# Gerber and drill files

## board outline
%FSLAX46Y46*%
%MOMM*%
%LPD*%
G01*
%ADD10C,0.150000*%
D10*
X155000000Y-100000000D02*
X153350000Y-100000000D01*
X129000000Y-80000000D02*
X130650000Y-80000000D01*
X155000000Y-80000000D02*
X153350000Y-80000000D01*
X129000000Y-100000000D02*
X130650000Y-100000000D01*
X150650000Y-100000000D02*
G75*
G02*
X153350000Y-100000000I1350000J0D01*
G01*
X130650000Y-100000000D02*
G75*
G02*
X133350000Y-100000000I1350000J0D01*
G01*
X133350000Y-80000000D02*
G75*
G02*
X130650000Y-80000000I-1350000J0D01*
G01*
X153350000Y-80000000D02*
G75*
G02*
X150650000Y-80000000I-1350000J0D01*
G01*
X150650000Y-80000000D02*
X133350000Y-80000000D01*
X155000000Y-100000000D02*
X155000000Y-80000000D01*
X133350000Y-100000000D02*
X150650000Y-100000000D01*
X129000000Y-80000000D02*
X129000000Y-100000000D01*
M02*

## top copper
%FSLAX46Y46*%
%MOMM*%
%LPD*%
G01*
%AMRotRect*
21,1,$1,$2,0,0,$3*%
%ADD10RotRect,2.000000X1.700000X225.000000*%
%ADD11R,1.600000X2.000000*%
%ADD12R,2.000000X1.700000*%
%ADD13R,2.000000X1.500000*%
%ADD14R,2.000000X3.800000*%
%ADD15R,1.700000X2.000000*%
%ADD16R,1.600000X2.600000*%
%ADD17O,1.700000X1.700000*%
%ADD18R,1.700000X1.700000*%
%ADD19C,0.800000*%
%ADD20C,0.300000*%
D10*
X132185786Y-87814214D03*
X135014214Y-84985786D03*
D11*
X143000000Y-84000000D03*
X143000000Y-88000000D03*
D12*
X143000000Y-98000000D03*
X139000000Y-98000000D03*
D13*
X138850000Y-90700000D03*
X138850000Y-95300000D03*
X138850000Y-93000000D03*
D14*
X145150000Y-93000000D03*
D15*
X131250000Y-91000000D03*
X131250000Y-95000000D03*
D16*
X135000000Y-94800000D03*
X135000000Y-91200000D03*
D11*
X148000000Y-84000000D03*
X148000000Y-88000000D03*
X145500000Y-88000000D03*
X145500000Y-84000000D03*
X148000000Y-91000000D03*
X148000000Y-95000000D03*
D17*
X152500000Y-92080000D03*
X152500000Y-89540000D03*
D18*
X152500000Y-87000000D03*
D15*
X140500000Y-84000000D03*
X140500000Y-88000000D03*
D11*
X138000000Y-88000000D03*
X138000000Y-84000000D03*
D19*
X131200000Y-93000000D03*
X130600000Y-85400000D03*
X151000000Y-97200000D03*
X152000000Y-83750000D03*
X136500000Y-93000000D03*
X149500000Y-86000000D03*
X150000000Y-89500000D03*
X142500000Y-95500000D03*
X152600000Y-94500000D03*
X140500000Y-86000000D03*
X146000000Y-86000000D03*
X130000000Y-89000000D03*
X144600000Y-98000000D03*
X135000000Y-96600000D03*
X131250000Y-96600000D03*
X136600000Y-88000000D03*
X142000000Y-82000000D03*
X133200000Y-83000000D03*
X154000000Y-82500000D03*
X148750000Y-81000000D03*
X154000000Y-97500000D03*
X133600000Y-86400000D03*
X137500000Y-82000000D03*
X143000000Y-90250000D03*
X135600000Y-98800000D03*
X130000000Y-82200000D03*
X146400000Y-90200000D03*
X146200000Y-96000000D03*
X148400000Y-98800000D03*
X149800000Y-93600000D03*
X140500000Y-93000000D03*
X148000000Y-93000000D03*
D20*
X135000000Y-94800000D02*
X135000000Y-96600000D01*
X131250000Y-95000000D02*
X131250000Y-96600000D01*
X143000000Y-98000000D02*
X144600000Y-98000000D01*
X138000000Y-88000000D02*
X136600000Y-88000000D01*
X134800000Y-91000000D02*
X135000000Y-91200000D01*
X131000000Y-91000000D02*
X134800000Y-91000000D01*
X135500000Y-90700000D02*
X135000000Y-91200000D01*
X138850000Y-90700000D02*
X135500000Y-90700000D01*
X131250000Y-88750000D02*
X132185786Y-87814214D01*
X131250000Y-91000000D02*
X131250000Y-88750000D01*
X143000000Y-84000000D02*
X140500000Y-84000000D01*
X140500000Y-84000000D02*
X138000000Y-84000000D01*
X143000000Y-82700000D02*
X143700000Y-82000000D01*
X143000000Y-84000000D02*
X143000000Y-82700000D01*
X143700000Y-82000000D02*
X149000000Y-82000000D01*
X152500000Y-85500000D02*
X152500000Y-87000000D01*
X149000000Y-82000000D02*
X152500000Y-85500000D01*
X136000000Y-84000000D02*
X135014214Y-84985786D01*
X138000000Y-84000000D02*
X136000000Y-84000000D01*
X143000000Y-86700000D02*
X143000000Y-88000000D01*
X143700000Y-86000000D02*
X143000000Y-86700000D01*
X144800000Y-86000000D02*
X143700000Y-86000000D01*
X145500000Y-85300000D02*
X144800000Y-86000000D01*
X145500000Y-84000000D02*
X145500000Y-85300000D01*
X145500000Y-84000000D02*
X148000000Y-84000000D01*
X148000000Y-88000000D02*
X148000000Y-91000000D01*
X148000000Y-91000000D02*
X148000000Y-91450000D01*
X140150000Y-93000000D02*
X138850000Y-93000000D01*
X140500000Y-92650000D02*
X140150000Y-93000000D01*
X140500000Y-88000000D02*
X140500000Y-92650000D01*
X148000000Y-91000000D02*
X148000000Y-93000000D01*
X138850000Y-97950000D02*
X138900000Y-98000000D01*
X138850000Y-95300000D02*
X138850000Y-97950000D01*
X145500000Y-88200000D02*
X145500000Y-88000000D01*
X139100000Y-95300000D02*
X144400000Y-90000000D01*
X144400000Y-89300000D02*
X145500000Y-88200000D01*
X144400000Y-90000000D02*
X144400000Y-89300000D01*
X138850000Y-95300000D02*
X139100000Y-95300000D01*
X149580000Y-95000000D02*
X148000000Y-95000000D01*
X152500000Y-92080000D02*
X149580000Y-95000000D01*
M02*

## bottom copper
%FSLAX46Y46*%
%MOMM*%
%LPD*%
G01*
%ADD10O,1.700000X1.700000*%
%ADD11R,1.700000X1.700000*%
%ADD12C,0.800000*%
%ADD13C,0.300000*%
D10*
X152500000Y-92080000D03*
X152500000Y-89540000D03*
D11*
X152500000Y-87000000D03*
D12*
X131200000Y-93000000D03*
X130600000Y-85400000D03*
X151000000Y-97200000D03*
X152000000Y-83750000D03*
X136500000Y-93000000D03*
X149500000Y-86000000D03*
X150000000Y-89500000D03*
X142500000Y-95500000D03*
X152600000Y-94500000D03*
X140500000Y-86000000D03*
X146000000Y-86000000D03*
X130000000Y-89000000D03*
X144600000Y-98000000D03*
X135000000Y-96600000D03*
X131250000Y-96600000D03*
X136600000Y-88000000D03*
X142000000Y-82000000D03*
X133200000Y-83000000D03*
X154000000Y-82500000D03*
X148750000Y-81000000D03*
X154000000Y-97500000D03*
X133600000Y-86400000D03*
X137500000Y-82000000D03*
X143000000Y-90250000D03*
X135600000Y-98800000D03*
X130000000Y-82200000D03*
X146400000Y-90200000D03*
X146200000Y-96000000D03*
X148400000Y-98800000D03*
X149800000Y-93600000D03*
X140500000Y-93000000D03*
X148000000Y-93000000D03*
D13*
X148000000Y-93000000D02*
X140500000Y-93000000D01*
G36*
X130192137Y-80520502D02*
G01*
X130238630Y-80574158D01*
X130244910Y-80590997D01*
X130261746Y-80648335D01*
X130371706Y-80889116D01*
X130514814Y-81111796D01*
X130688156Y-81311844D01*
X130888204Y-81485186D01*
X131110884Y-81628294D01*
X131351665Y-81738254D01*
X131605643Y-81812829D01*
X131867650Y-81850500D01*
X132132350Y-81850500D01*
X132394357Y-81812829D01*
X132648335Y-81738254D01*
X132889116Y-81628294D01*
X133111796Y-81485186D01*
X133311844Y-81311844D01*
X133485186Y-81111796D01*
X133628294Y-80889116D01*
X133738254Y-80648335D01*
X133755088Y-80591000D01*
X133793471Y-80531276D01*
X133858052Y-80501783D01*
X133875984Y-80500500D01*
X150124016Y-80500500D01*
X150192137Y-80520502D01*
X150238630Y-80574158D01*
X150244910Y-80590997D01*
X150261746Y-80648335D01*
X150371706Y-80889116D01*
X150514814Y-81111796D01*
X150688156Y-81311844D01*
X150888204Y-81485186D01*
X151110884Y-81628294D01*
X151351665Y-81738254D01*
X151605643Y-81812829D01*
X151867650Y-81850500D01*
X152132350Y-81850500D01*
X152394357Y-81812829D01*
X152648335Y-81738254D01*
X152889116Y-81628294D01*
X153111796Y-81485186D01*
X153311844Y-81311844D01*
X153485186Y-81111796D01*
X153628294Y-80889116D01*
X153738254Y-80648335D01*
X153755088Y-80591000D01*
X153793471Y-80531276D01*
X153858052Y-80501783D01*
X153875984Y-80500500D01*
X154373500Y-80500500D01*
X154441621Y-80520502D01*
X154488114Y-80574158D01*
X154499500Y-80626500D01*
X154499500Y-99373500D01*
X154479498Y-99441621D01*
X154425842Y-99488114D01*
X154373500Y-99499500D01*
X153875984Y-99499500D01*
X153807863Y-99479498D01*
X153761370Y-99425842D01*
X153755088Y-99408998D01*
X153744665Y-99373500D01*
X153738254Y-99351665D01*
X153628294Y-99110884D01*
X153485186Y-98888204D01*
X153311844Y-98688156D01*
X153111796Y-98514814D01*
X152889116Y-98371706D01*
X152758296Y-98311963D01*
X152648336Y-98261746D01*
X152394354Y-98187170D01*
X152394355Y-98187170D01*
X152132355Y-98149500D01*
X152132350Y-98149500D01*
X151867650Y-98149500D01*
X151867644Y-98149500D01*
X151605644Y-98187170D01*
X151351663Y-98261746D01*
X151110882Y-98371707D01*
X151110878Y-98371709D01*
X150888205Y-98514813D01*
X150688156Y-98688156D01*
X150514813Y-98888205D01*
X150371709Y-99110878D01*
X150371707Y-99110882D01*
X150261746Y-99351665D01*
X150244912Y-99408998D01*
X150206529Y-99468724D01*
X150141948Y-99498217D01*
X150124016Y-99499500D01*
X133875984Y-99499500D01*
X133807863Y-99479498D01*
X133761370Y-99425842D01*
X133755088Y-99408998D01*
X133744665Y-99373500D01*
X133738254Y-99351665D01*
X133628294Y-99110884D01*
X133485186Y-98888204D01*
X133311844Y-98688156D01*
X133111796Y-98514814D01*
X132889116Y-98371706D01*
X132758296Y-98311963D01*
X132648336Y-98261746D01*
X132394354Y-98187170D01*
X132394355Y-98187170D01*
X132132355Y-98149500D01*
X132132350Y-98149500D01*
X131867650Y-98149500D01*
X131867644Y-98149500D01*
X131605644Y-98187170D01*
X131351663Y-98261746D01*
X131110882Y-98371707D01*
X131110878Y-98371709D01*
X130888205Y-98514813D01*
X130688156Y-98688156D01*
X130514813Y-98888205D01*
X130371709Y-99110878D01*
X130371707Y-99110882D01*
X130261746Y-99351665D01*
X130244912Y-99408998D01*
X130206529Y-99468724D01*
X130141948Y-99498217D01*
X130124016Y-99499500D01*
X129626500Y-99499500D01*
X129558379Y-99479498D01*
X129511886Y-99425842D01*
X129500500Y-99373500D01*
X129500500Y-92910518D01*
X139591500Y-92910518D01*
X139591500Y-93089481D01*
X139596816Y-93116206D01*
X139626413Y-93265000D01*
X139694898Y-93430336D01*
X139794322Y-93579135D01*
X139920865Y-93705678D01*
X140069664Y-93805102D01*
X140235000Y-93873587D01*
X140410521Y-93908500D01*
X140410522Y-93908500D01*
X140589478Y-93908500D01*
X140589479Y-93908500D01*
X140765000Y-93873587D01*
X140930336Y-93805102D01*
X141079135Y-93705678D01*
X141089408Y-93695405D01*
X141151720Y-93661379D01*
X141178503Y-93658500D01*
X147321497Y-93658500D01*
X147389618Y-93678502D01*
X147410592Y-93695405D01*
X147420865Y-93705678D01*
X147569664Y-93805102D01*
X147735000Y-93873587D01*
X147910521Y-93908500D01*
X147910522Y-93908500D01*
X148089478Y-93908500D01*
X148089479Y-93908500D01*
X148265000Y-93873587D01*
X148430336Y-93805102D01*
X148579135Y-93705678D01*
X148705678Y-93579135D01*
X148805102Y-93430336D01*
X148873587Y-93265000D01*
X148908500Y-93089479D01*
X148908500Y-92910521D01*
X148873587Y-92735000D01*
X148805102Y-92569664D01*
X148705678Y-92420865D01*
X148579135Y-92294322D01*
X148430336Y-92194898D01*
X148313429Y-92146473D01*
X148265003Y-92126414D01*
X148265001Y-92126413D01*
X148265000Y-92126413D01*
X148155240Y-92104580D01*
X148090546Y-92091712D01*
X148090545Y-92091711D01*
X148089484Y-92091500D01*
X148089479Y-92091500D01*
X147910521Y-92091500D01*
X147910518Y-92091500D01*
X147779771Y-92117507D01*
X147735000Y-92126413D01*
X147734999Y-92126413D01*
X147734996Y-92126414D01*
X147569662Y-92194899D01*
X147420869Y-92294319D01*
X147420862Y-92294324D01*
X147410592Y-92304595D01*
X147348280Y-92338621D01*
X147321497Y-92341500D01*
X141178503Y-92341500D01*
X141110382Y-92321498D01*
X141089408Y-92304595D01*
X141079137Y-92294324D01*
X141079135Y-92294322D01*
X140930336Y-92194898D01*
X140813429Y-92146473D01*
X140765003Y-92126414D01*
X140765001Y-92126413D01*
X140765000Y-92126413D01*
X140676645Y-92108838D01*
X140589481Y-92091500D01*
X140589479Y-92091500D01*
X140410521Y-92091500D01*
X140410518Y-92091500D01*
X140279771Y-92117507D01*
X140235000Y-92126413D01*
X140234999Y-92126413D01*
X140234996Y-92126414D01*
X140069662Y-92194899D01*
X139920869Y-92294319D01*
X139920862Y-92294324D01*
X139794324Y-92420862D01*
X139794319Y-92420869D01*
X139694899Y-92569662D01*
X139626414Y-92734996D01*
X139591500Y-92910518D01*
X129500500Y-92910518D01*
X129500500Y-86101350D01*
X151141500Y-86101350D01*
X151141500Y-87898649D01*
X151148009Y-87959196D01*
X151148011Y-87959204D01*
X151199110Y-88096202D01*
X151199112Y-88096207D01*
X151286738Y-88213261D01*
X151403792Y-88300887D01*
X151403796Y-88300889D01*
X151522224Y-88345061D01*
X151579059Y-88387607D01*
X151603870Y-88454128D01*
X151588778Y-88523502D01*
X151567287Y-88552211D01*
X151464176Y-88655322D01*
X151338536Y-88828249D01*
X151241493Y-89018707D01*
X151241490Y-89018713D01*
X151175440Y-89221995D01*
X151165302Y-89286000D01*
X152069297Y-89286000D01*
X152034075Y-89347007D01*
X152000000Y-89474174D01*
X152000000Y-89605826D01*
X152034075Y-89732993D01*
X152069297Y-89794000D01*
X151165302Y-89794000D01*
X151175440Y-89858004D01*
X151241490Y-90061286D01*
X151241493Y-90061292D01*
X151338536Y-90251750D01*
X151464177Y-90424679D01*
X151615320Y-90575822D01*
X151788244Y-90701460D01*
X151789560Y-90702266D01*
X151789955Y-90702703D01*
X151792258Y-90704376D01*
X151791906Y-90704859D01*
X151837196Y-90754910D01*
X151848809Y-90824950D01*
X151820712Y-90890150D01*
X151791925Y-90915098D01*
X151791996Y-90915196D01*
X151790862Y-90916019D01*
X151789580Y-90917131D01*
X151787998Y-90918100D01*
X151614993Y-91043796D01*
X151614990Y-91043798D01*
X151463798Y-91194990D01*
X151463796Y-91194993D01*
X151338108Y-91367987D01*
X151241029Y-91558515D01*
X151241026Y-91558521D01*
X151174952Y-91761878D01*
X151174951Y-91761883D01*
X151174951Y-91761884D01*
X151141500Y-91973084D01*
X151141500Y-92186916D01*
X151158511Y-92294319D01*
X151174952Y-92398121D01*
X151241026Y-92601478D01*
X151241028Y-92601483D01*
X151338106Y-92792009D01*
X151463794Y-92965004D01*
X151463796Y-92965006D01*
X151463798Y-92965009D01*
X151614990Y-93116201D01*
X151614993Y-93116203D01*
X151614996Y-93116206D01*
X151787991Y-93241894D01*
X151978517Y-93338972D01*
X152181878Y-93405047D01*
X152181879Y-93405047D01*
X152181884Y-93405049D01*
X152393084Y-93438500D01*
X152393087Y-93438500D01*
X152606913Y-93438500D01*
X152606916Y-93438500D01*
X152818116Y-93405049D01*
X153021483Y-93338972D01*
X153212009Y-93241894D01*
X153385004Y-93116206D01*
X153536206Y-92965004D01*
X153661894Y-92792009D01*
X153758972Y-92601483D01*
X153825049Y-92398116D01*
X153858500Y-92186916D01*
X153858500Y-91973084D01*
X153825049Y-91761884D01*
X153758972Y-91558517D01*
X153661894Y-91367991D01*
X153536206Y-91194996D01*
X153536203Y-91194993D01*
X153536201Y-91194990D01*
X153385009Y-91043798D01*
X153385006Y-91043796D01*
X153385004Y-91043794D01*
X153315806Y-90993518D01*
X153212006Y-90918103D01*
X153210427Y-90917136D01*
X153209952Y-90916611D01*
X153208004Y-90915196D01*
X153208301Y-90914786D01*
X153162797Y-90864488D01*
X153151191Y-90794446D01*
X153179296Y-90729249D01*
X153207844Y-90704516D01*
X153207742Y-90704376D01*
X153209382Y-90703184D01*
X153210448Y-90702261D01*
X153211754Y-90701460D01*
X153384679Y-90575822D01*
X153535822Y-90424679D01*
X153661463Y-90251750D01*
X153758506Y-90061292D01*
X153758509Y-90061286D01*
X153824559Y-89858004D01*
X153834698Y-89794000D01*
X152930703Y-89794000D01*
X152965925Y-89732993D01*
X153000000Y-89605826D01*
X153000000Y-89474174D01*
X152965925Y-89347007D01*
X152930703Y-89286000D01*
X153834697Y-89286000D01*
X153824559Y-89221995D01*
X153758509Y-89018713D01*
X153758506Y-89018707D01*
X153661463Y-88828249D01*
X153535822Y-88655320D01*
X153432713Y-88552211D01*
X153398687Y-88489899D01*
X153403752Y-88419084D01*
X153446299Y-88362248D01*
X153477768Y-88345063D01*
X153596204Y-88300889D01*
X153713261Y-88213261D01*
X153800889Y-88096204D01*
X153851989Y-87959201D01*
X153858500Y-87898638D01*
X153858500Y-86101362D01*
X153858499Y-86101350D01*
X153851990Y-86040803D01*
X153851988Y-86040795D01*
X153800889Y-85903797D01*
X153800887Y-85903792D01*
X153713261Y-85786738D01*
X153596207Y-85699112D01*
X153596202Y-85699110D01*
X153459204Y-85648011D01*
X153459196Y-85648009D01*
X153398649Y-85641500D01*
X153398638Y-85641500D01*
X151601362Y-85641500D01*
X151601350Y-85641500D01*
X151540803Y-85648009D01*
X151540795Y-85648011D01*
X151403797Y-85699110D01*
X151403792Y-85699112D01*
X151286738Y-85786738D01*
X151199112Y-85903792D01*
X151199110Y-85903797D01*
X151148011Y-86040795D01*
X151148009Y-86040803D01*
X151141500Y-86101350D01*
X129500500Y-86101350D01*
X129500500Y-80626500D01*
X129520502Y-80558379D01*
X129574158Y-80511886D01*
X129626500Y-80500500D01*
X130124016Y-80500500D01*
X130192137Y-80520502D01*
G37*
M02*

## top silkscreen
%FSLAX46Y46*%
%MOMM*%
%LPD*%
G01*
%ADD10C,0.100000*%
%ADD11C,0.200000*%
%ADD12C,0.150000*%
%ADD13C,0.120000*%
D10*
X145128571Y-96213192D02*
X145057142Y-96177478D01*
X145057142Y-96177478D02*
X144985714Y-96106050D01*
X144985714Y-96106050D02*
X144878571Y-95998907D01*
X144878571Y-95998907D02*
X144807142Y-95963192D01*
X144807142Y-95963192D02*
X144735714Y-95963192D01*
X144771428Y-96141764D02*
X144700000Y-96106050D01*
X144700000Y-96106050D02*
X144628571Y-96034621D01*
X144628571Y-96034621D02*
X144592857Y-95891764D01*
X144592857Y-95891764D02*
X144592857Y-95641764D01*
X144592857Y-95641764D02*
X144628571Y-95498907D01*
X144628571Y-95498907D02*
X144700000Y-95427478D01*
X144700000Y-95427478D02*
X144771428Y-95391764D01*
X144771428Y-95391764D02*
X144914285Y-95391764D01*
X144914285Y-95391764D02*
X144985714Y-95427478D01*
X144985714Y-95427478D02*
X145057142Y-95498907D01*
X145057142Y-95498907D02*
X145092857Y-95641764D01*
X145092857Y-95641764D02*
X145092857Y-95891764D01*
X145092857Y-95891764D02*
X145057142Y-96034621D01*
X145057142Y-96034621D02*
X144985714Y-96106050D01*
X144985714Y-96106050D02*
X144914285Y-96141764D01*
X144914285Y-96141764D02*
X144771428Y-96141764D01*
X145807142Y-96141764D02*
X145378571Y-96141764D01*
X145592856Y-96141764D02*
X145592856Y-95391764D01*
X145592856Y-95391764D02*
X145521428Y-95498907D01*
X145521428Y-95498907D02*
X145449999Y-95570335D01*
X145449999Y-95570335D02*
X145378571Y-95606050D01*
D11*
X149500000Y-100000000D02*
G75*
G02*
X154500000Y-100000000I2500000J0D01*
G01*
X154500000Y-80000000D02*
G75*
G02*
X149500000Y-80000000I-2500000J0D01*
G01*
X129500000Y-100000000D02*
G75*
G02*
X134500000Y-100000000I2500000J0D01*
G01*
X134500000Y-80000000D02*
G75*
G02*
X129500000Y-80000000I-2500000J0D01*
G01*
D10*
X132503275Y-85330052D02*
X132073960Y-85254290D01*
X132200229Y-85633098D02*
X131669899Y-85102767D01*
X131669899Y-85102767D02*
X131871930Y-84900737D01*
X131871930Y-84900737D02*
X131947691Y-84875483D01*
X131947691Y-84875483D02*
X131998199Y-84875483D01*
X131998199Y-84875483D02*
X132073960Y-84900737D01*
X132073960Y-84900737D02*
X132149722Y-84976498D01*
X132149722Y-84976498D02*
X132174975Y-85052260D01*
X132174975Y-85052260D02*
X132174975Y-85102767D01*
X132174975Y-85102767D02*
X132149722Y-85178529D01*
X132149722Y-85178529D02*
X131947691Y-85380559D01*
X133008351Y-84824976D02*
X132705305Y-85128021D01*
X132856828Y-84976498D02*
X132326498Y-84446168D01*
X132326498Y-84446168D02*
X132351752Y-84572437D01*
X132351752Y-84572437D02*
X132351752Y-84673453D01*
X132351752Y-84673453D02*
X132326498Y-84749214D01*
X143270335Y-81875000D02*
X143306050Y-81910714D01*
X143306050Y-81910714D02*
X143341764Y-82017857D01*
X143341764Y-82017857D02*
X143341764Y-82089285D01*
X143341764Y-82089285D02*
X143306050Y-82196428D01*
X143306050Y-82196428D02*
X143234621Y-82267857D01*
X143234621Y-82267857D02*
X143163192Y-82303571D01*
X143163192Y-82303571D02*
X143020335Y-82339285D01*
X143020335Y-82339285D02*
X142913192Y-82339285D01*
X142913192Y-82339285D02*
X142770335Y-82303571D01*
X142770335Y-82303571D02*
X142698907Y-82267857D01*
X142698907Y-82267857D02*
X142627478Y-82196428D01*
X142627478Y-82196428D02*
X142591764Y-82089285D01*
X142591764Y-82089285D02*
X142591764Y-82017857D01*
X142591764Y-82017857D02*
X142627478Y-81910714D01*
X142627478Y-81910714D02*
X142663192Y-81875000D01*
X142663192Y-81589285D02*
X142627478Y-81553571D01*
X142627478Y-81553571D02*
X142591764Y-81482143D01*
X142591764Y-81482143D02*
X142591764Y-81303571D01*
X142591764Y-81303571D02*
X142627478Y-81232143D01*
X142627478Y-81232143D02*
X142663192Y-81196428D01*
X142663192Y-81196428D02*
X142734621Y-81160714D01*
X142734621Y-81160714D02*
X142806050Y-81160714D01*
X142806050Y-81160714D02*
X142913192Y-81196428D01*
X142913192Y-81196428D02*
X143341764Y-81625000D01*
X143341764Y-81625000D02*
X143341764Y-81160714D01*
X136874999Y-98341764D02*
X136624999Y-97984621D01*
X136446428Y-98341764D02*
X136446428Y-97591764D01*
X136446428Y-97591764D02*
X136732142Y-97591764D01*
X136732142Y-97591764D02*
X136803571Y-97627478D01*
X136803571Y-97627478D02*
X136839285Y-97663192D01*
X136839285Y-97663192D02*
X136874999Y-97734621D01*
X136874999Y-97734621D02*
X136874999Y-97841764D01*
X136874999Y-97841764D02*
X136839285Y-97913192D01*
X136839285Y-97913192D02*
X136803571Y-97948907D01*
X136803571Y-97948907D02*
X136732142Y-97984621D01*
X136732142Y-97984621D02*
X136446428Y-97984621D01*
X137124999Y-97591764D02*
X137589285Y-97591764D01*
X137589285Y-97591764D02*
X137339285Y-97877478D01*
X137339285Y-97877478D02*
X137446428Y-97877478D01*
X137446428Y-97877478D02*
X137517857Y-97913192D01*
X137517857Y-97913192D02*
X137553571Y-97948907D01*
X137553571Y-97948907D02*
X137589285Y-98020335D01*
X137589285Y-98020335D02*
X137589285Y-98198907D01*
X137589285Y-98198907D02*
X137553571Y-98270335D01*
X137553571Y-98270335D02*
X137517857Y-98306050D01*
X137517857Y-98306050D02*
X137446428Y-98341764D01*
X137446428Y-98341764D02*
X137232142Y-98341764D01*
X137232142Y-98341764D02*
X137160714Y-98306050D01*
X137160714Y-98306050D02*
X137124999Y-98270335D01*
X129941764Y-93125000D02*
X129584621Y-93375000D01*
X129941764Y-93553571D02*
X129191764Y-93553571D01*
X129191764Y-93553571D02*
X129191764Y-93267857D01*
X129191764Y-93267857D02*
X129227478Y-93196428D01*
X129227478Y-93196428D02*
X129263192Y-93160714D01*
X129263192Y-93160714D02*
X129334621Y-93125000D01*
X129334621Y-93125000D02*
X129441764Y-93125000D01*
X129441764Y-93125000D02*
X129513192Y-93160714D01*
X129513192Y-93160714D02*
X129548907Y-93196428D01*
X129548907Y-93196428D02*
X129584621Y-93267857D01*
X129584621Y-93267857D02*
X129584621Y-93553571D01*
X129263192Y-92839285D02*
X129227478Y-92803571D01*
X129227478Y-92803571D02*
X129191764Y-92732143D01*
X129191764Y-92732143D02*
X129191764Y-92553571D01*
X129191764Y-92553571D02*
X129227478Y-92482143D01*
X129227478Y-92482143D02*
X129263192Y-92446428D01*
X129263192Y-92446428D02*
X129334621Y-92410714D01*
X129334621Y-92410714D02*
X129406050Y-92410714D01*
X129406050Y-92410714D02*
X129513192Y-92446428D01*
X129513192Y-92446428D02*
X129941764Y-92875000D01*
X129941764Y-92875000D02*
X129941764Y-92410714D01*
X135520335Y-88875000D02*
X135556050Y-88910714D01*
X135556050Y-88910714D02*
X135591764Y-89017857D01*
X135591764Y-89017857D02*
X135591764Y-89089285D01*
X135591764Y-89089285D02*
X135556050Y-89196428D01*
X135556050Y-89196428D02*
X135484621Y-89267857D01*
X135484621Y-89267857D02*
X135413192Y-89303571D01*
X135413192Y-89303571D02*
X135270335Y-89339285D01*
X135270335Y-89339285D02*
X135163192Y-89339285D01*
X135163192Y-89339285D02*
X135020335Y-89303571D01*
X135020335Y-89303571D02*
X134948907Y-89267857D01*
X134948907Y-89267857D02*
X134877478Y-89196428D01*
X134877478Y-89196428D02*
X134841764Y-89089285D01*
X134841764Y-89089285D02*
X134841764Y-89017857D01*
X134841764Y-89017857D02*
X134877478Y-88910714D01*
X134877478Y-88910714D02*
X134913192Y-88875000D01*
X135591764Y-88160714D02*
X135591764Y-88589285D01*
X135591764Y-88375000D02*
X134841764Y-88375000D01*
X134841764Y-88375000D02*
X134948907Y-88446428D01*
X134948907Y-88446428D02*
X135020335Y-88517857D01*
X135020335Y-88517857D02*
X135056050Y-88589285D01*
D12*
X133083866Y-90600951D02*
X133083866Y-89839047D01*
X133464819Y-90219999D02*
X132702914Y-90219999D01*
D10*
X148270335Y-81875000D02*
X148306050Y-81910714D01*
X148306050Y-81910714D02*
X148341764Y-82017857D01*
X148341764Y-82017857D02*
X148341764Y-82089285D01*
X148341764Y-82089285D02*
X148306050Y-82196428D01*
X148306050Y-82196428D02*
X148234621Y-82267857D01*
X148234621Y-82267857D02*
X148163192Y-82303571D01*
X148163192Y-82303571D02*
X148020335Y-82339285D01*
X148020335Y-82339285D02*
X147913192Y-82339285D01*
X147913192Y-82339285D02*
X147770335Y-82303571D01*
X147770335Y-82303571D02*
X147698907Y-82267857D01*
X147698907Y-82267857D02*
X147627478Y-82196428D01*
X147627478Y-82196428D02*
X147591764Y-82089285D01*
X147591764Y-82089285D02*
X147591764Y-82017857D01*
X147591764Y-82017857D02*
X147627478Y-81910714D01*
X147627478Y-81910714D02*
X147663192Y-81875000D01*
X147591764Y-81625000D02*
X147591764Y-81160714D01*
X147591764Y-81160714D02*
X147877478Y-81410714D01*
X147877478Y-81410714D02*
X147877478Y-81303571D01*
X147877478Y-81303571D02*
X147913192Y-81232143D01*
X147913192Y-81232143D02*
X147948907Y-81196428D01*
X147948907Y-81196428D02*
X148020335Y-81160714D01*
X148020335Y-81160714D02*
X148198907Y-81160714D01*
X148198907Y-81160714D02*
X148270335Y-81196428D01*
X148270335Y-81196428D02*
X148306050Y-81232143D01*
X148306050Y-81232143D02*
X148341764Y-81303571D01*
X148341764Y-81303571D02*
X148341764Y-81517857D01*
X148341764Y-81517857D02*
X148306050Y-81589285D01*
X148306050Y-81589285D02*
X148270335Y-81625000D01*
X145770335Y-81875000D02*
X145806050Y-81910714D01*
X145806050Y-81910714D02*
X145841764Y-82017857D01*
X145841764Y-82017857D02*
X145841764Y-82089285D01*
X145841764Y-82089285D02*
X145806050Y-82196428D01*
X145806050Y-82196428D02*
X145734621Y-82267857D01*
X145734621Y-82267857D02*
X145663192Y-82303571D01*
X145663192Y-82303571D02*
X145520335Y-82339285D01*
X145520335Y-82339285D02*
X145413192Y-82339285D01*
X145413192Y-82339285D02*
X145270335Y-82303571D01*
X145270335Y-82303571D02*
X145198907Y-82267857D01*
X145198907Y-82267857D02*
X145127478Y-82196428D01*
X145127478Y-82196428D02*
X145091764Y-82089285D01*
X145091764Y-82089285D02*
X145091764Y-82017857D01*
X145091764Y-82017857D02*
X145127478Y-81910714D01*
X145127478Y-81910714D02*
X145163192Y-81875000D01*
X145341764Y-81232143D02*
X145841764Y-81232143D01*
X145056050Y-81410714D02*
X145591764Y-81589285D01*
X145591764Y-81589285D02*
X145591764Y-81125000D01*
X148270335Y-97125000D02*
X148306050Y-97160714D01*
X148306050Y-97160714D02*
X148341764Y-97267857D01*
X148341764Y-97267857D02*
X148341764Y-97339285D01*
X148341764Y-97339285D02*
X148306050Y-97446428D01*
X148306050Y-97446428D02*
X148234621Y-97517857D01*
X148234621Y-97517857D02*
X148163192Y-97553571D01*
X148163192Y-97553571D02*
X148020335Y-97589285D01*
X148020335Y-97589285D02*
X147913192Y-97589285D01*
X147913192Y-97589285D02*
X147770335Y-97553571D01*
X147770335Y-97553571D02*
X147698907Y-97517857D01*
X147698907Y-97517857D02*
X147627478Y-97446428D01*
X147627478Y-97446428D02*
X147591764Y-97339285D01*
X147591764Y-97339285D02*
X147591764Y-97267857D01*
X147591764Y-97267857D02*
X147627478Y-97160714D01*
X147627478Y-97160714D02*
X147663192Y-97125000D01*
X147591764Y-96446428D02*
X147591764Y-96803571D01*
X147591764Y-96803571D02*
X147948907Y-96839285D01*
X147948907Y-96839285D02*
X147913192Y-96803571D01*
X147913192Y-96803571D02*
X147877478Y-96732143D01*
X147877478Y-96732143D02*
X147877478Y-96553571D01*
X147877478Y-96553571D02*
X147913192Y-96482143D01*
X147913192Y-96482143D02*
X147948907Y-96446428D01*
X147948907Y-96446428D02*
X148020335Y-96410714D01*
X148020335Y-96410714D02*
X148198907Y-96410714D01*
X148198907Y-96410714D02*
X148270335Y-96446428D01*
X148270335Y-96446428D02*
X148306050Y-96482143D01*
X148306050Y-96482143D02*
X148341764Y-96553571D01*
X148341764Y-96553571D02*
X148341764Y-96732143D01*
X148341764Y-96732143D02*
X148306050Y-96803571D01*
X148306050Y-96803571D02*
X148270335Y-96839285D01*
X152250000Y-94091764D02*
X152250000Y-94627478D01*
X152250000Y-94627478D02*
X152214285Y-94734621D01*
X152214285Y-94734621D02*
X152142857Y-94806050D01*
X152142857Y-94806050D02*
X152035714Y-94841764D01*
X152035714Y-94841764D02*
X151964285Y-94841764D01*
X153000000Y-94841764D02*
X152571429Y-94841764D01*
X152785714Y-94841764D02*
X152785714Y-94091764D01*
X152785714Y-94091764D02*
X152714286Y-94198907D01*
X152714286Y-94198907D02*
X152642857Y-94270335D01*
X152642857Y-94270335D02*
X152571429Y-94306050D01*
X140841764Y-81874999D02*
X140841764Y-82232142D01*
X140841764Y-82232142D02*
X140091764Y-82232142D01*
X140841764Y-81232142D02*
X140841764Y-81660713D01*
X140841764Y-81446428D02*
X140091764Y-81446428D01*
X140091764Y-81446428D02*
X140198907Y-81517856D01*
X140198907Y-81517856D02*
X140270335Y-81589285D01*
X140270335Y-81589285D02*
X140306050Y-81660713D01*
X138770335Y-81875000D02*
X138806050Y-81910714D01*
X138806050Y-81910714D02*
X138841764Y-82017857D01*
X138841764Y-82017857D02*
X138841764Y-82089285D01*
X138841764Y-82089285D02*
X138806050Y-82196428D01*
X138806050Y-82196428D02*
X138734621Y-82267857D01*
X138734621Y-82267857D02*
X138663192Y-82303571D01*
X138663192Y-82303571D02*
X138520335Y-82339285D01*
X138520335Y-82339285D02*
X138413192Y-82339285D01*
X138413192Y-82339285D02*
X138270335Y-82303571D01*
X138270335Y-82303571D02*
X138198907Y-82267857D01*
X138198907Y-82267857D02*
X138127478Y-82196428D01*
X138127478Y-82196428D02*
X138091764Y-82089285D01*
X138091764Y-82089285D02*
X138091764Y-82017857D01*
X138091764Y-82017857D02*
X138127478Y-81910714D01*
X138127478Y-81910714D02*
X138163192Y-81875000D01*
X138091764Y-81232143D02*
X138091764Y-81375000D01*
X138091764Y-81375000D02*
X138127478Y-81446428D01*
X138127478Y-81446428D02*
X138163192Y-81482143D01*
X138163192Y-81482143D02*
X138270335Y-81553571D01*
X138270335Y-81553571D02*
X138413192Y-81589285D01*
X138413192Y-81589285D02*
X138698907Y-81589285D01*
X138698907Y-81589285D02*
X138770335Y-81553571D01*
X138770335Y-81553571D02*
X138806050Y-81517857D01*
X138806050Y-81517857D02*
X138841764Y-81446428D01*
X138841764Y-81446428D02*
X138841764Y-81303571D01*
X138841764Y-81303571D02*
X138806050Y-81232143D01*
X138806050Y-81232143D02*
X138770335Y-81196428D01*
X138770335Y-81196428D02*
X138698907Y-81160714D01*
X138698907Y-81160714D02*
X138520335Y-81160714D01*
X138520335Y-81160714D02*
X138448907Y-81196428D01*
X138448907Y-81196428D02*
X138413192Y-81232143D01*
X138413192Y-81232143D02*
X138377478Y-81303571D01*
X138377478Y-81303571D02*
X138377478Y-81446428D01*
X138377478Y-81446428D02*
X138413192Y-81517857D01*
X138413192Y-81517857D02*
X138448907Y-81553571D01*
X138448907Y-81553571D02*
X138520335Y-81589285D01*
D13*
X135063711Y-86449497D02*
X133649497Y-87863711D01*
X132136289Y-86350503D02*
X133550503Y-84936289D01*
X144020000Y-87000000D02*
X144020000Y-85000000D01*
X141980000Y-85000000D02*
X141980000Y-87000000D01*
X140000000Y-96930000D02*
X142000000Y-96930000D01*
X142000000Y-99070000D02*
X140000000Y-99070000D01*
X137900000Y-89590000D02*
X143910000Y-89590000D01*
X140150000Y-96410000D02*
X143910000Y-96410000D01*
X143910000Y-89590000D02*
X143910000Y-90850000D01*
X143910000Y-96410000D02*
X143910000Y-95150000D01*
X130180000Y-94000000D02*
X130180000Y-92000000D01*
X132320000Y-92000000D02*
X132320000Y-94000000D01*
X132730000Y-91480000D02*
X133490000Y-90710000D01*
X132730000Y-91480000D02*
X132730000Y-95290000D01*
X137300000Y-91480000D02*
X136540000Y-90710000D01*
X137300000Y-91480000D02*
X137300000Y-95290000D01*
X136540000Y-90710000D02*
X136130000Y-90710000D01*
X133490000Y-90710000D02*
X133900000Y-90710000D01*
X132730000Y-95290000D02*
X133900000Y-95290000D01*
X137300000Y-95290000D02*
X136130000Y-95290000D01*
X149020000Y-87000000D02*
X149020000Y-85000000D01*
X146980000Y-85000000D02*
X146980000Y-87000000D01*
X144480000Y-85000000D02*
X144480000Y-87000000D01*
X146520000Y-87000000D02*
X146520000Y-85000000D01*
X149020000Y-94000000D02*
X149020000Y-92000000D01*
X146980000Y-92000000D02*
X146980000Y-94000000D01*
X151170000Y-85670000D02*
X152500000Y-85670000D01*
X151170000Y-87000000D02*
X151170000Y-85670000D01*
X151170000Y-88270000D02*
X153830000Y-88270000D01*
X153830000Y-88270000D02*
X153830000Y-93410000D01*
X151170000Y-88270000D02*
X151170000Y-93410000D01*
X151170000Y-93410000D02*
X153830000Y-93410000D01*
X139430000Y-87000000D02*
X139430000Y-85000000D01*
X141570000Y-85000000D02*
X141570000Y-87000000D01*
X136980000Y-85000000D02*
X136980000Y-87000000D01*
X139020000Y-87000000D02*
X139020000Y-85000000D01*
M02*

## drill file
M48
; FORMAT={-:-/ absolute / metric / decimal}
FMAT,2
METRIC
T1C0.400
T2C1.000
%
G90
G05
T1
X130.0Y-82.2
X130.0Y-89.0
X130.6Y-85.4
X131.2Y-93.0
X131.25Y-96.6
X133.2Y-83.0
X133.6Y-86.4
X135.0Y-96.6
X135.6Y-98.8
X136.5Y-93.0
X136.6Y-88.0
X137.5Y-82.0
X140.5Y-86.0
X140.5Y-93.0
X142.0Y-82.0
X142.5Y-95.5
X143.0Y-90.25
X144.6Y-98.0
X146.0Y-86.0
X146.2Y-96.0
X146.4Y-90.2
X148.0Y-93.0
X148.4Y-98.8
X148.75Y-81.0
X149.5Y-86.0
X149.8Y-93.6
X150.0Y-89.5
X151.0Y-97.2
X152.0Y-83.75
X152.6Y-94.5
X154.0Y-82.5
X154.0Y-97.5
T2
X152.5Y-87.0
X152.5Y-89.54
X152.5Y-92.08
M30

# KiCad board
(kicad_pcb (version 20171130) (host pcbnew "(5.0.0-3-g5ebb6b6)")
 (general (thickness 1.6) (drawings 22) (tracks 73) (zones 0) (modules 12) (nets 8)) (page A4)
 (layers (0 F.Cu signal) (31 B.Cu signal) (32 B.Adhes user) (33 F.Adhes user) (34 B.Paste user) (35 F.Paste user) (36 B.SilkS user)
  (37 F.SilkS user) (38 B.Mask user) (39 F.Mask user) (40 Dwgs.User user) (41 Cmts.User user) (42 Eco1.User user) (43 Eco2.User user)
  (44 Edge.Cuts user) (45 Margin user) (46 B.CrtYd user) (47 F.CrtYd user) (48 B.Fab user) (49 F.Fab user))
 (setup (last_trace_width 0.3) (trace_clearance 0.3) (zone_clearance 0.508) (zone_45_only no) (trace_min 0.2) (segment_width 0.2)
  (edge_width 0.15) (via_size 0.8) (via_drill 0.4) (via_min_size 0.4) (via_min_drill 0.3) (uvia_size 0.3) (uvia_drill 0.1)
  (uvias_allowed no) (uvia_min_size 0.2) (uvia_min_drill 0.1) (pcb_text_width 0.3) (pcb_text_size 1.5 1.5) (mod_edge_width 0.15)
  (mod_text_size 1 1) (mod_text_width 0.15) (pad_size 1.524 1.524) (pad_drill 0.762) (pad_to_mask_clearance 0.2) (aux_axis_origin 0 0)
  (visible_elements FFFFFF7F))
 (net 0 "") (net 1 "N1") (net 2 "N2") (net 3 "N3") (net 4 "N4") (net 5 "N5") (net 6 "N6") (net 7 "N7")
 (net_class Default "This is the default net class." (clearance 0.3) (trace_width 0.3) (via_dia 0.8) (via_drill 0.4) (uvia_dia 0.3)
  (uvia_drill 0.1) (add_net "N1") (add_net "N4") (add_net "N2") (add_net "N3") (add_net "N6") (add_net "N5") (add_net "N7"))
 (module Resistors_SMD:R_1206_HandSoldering (layer F.Cu) (at 133.6 86.4 225)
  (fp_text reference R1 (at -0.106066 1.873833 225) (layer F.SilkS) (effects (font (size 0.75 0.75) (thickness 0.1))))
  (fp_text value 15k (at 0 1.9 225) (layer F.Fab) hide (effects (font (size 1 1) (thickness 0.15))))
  (fp_line (start -1 -1.07) (end 1 -1.07) (layer F.SilkS) (width 0.12))
  (fp_line (start 1 1.07) (end -1 1.07) (layer F.SilkS) (width 0.12))
  (pad 2 smd rect (at 2.000001 0 225) (size 2 1.7) (layers F.Cu F.Paste F.Mask) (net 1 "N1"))
  (pad 1 smd rect (at -2.000001 0 225) (size 2 1.7) (layers F.Cu F.Paste F.Mask) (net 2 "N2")))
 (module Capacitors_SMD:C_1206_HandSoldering (layer F.Cu) (at 143 86 270)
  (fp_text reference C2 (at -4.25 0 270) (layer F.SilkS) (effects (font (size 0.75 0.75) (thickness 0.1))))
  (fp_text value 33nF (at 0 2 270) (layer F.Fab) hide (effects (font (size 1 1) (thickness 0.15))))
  (fp_line (start 1 -1.02) (end -1 -1.02) (layer F.SilkS) (width 0.12))
  (fp_line (start -1 1.02) (end 1 1.02) (layer F.SilkS) (width 0.12))
  (pad 1 smd rect (at -2 0 270) (size 2 1.6) (layers F.Cu F.Paste F.Mask) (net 2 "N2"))
  (pad 2 smd rect (at 2 0 270) (size 2 1.6) (layers F.Cu F.Paste F.Mask) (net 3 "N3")))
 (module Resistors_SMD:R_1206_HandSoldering (layer F.Cu) (at 141 98)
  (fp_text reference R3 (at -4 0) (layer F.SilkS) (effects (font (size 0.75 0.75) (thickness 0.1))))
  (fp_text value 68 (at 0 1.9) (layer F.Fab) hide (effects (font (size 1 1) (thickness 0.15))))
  (fp_line (start -1 -1.07) (end 1 -1.07) (layer F.SilkS) (width 0.12))
  (fp_line (start 1 1.07) (end -1 1.07) (layer F.SilkS) (width 0.12))
  (pad 2 smd rect (at 2 0) (size 2 1.7) (layers F.Cu F.Paste F.Mask) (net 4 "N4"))
  (pad 1 smd rect (at -2 0) (size 2 1.7) (layers F.Cu F.Paste F.Mask) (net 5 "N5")))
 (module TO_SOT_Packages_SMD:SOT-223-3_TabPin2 (layer F.Cu) (at 142 93)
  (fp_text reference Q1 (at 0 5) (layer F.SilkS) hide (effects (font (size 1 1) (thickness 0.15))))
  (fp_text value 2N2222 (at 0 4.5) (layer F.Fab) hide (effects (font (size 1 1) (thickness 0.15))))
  (fp_line (start -4.1 -3.41) (end 1.91 -3.41) (layer F.SilkS) (width 0.12))
  (fp_line (start -1.85 3.41) (end 1.91 3.41) (layer F.SilkS) (width 0.12))
  (fp_line (start 1.91 -3.41) (end 1.91 -2.15) (layer F.SilkS) (width 0.12))
  (fp_line (start 1.91 3.41) (end 1.91 2.15) (layer F.SilkS) (width 0.12))
  (pad 1 smd rect (at -3.15 -2.3) (size 2 1.5) (layers F.Cu F.Paste F.Mask) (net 1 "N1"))
  (pad 3 smd rect (at -3.15 2.3) (size 2 1.5) (layers F.Cu F.Paste F.Mask) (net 5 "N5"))
  (pad 2 smd rect (at -3.15 0) (size 2 1.5) (layers F.Cu F.Paste F.Mask) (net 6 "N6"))
  (pad 2 smd rect (at 3.15 0) (size 2 3.8) (layers F.Cu F.Paste F.Mask) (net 6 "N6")))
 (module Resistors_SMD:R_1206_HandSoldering (layer F.Cu) (at 131.25 93 270)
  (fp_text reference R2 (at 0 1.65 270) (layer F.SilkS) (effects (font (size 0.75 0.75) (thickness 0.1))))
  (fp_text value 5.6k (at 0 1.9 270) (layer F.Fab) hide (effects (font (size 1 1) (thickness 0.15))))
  (fp_line (start 1 1.07) (end -1 1.07) (layer F.SilkS) (width 0.12))
  (fp_line (start -1 -1.07) (end 1 -1.07) (layer F.SilkS) (width 0.12))
  (pad 1 smd rect (at -2 0 270) (size 2 1.7) (layers F.Cu F.Paste F.Mask) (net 1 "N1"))
  (pad 2 smd rect (at 2 0 270) (size 2 1.7) (layers F.Cu F.Paste F.Mask) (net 4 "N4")))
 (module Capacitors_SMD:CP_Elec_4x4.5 (layer F.Cu) (at 135 93 270)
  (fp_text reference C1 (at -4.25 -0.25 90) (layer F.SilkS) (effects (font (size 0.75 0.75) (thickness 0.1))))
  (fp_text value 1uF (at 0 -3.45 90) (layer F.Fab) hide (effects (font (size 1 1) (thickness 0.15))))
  (fp_line (start -1.52 2.27) (end -2.29 1.51) (layer F.SilkS) (width 0.12))
  (fp_line (start -1.52 2.27) (end 2.29 2.27) (layer F.SilkS) (width 0.12))
  (fp_line (start -1.52 -2.3) (end -2.29 -1.54) (layer F.SilkS) (width 0.12))
  (fp_line (start -1.52 -2.3) (end 2.29 -2.3) (layer F.SilkS) (width 0.12))
  (fp_line (start -2.29 -1.54) (end -2.29 -1.13) (layer F.SilkS) (width 0.12))
  (fp_line (start -2.29 1.51) (end -2.29 1.1) (layer F.SilkS) (width 0.12))
  (fp_line (start 2.29 2.27) (end 2.29 1.1) (layer F.SilkS) (width 0.12))
  (fp_line (start 2.29 -2.3) (end 2.29 -1.13) (layer F.SilkS) (width 0.12))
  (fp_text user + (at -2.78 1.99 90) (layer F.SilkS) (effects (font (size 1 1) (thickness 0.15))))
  (pad 2 smd rect (at 1.8 0 90) (size 2.6 1.6) (layers F.Cu F.Paste F.Mask) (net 4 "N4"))
  (pad 1 smd rect (at -1.8 0 90) (size 2.6 1.6) (layers F.Cu F.Paste F.Mask) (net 1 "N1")))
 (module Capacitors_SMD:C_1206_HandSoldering (layer F.Cu) (at 148 86 90)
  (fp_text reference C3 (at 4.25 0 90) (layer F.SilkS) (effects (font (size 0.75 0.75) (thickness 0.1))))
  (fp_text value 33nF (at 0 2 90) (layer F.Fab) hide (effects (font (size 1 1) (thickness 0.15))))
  (fp_line (start -1 1.02) (end 1 1.02) (layer F.SilkS) (width 0.12))
  (fp_line (start 1 -1.02) (end -1 -1.02) (layer F.SilkS) (width 0.12))
  (pad 2 smd rect (at 2 0 90) (size 2 1.6) (layers F.Cu F.Paste F.Mask) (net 3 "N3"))
  (pad 1 smd rect (at -2 0 90) (size 2 1.6) (layers F.Cu F.Paste F.Mask) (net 6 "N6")))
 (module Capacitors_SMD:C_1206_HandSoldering (layer F.Cu) (at 145.5 86 90)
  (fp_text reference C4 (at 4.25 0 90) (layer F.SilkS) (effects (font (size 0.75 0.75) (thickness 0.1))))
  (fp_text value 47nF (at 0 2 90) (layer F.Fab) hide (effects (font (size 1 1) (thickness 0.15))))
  (fp_line (start 1 -1.02) (end -1 -1.02) (layer F.SilkS) (width 0.12))
  (fp_line (start -1 1.02) (end 1 1.02) (layer F.SilkS) (width 0.12))
  (pad 1 smd rect (at -2 0 90) (size 2 1.6) (layers F.Cu F.Paste F.Mask) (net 5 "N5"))
  (pad 2 smd rect (at 2 0 90) (size 2 1.6) (layers F.Cu F.Paste F.Mask) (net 3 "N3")))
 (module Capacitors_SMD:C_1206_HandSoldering (layer F.Cu) (at 148 93 90)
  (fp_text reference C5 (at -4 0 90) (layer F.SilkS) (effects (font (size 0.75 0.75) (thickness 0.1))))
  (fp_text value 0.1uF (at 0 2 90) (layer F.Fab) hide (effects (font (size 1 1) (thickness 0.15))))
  (fp_line (start -1 1.02) (end 1 1.02) (layer F.SilkS) (width 0.12))
  (fp_line (start 1 -1.02) (end -1 -1.02) (layer F.SilkS) (width 0.12))
  (pad 2 smd rect (at 2 0 90) (size 2 1.6) (layers F.Cu F.Paste F.Mask) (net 6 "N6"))
  (pad 1 smd rect (at -2 0 90) (size 2 1.6) (layers F.Cu F.Paste F.Mask) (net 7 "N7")))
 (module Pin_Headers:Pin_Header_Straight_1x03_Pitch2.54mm (layer F.Cu) (at 152.5 87)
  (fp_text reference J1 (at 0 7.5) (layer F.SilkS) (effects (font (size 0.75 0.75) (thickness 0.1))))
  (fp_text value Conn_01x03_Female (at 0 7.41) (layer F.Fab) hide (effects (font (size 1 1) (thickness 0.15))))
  (fp_line (start -1.33 -1.33) (end 0 -1.33) (layer F.SilkS) (width 0.12))
  (fp_line (start -1.33 0) (end -1.33 -1.33) (layer F.SilkS) (width 0.12))
  (fp_line (start -1.33 1.27) (end 1.33 1.27) (layer F.SilkS) (width 0.12))
  (fp_line (start 1.33 1.27) (end 1.33 6.41) (layer F.SilkS) (width 0.12))
  (fp_line (start -1.33 1.27) (end -1.33 6.41) (layer F.SilkS) (width 0.12))
  (fp_line (start -1.33 6.41) (end 1.33 6.41) (layer F.SilkS) (width 0.12))
  (pad 3 thru_hole oval (at 0 5.08) (size 1.7 1.7) (drill 1) (layers *.Cu *.Mask) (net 7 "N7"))
  (pad 2 thru_hole oval (at 0 2.54) (size 1.7 1.7) (drill 1) (layers *.Cu *.Mask) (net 4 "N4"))
  (pad 1 thru_hole rect (at 0 0) (size 1.7 1.7) (drill 1) (layers *.Cu *.Mask) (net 2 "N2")))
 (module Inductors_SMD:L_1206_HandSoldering (layer F.Cu) (at 140.5 86 90)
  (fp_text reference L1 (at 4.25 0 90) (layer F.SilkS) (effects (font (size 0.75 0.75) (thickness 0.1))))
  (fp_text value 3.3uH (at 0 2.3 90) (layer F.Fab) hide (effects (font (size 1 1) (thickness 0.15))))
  (fp_line (start -1 -1.07) (end 1 -1.07) (layer F.SilkS) (width 0.12))
  (fp_line (start 1 1.07) (end -1 1.07) (layer F.SilkS) (width 0.12))
  (pad 2 smd rect (at 2 0 90) (size 2 1.7) (layers F.Cu F.Paste F.Mask) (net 2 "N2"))
  (pad 1 smd rect (at -2 0 90) (size 2 1.7) (layers F.Cu F.Paste F.Mask) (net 6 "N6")))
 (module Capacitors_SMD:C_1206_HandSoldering (layer F.Cu) (at 138 86 270)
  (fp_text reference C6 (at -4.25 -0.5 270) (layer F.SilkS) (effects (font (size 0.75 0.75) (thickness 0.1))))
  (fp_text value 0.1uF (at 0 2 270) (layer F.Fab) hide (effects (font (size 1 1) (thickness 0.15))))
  (fp_line (start -1 1.02) (end 1 1.02) (layer F.SilkS) (width 0.12))
  (fp_line (start 1 -1.02) (end -1 -1.02) (layer F.SilkS) (width 0.12))
  (pad 2 smd rect (at 2 0 270) (size 2 1.6) (layers F.Cu F.Paste F.Mask) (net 4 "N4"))
  (pad 1 smd rect (at -2 0 270) (size 2 1.6) (layers F.Cu F.Paste F.Mask) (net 2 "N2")))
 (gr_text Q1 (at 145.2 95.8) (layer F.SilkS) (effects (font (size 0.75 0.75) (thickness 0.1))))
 (gr_line (start 155 100) (end 153.35 100) (layer Edge.Cuts) (width 0.15))
 (gr_line (start 129 80) (end 130.65 80) (layer Edge.Cuts) (width 0.15))
 (gr_line (start 155 80) (end 153.35 80) (layer Edge.Cuts) (width 0.15))
 (gr_line (start 129 100) (end 130.65 100) (layer Edge.Cuts) (width 0.15))
 (gr_arc (start 152 100) (end 153.35 100) (angle -180) (layer Edge.Cuts) (width 0.15))
 (gr_arc (start 132 100) (end 133.35 100) (angle -180) (layer Edge.Cuts) (width 0.15))
 (gr_arc (start 132 80) (end 130.65 80) (angle -180) (layer Edge.Cuts) (width 0.15))
 (gr_arc (start 152 80) (end 150.65 80) (angle -180) (layer Edge.Cuts) (width 0.15))
 (gr_arc (start 152 100) (end 154.5 100) (angle -180) (layer F.SilkS) (width 0.2))
 (gr_arc (start 152 80) (end 149.5 80) (angle -180) (layer F.SilkS) (width 0.2))
 (gr_arc (start 132 100) (end 134.5 100) (angle -180) (layer F.SilkS) (width 0.2))
 (gr_arc (start 132 80) (end 129.5 80) (angle -180) (layer F.SilkS) (width 0.2))
 (gr_line (start 150.65 80) (end 133.35 80) (layer Edge.Cuts) (width 0.15))
 (gr_line (start 155 100) (end 155 80) (layer Edge.Cuts) (width 0.15))
 (gr_line (start 133.35 100) (end 150.65 100) (layer Edge.Cuts) (width 0.15))
 (gr_line (start 129 80) (end 129 100) (layer Edge.Cuts) (width 0.15))
 (via (at 131.2 93) (size 0.8) (drill 0.4) (layers F.Cu B.Cu) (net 4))
 (via (at 130.6 85.4) (size 0.8) (drill 0.4) (layers F.Cu B.Cu) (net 4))
 (via (at 151 97.2) (size 0.8) (drill 0.4) (layers F.Cu B.Cu) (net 4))
 (via (at 152 83.75) (size 0.8) (drill 0.4) (layers F.Cu B.Cu) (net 4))
 (via (at 136.5 93) (size 0.8) (drill 0.4) (layers F.Cu B.Cu) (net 4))
 (via (at 149.5 86) (size 0.8) (drill 0.4) (layers F.Cu B.Cu) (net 4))
 (via (at 150 89.5) (size 0.8) (drill 0.4) (layers F.Cu B.Cu) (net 4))
 (via (at 142.5 95.5) (size 0.8) (drill 0.4) (layers F.Cu B.Cu) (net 4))
 (via (at 152.6 94.5) (size 0.8) (drill 0.4) (layers F.Cu B.Cu) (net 4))
 (via (at 140.5 86) (size 0.8) (drill 0.4) (layers F.Cu B.Cu) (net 4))
 (via (at 146 86) (size 0.8) (drill 0.4) (layers F.Cu B.Cu) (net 4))
 (via (at 130 89) (size 0.8) (drill 0.4) (layers F.Cu B.Cu) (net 4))
 (via (at 144.6 98) (size 0.8) (drill 0.4) (layers F.Cu B.Cu) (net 4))
 (via (at 135 96.6) (size 0.8) (drill 0.4) (layers F.Cu B.Cu) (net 4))
 (via (at 131.25 96.6) (size 0.8) (drill 0.4) (layers F.Cu B.Cu) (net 4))
 (via (at 136.6 88) (size 0.8) (drill 0.4) (layers F.Cu B.Cu) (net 4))
 (via (at 142 82) (size 0.8) (drill 0.4) (layers F.Cu B.Cu) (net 4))
 (via (at 133.2 83) (size 0.8) (drill 0.4) (layers F.Cu B.Cu) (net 4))
 (via (at 154 82.5) (size 0.8) (drill 0.4) (layers F.Cu B.Cu) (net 4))
 (via (at 148.75 81) (size 0.8) (drill 0.4) (layers F.Cu B.Cu) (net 4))
 (via (at 154 97.5) (size 0.8) (drill 0.4) (layers F.Cu B.Cu) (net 4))
 (via (at 133.6 86.4) (size 0.8) (drill 0.4) (layers F.Cu B.Cu) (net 4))
 (via (at 137.5 82) (size 0.8) (drill 0.4) (layers F.Cu B.Cu) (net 4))
 (via (at 143 90.25) (size 0.8) (drill 0.4) (layers F.Cu B.Cu) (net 4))
 (segment (start 135 94.8) (end 135 96.6) (width 0.3) (layer F.Cu) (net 4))
 (segment (start 131.25 95) (end 131.25 96.6) (width 0.3) (layer F.Cu) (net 4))
 (segment (start 143 98) (end 144.6 98) (width 0.3) (layer F.Cu) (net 4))
 (segment (start 138 88) (end 136.6 88) (width 0.3) (layer F.Cu) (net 4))
 (via (at 135.6 98.8) (size 0.8) (drill 0.4) (layers F.Cu B.Cu) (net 4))
 (via (at 130 82.2) (size 0.8) (drill 0.4) (layers F.Cu B.Cu) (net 4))
 (via (at 146.4 90.2) (size 0.8) (drill 0.4) (layers F.Cu B.Cu) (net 4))
 (via (at 146.2 96) (size 0.8) (drill 0.4) (layers F.Cu B.Cu) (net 4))
 (via (at 148.4 98.8) (size 0.8) (drill 0.4) (layers F.Cu B.Cu) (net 4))
 (via (at 149.8 93.6) (size 0.8) (drill 0.4) (layers F.Cu B.Cu) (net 4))
 (segment (start 134.8 91) (end 135 91.2) (width 0.3) (layer F.Cu) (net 1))
 (segment (start 131 91) (end 134.8 91) (width 0.3) (layer F.Cu) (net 1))
 (segment (start 135.5 90.7) (end 135 91.2) (width 0.3) (layer F.Cu) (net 1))
 (segment (start 138.85 90.7) (end 135.5 90.7) (width 0.3) (layer F.Cu) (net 1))
 (segment (start 131.25 88.75) (end 132.185786 87.814214) (width 0.3) (layer F.Cu) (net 1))
 (segment (start 131.25 91) (end 131.25 88.75) (width 0.3) (layer F.Cu) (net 1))
 (segment (start 143 84) (end 140.5 84) (width 0.3) (layer F.Cu) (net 2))
 (segment (start 140.5 84) (end 138 84) (width 0.3) (layer F.Cu) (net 2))
 (segment (start 143 82.7) (end 143.7 82) (width 0.3) (layer F.Cu) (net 2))
 (segment (start 143 84) (end 143 82.7) (width 0.3) (layer F.Cu) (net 2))
 (segment (start 143.7 82) (end 149 82) (width 0.3) (layer F.Cu) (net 2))
 (segment (start 152.5 85.5) (end 152.5 87) (width 0.3) (layer F.Cu) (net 2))
 (segment (start 149 82) (end 152.5 85.5) (width 0.3) (layer F.Cu) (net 2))
 (segment (start 136 84) (end 135.014214 84.985786) (width 0.3) (layer F.Cu) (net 2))
 (segment (start 138 84) (end 136 84) (width 0.3) (layer F.Cu) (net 2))
 (segment (start 143 86.7) (end 143 88) (width 0.3) (layer F.Cu) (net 3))
 (segment (start 143.7 86) (end 143 86.7) (width 0.3) (layer F.Cu) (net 3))
 (segment (start 144.8 86) (end 143.7 86) (width 0.3) (layer F.Cu) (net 3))
 (segment (start 145.5 85.3) (end 144.8 86) (width 0.3) (layer F.Cu) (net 3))
 (segment (start 145.5 84) (end 145.5 85.3) (width 0.3) (layer F.Cu) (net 3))
 (segment (start 145.5 84) (end 148 84) (width 0.3) (layer F.Cu) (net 3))
 (via (at 140.5 93) (size 0.8) (drill 0.4) (layers F.Cu B.Cu) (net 6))
 (via (at 148 93) (size 0.8) (drill 0.4) (layers F.Cu B.Cu) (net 6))
 (segment (start 148 88) (end 148 91) (width 0.3) (layer F.Cu) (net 6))
 (segment (start 148 91) (end 148 91.45) (width 0.3) (layer F.Cu) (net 6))
 (segment (start 140.15 93) (end 138.85 93) (width 0.3) (layer F.Cu) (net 6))
 (segment (start 140.5 92.65) (end 140.15 93) (width 0.3) (layer F.Cu) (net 6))
 (segment (start 140.5 88) (end 140.5 92.65) (width 0.3) (layer F.Cu) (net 6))
 (segment (start 148 91) (end 148 93) (width 0.3) (layer F.Cu) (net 6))
 (segment (start 148 93) (end 140.5 93) (width 0.3) (layer B.Cu) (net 6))
 (segment (start 138.85 97.95) (end 138.9 98) (width 0.3) (layer F.Cu) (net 5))
 (segment (start 138.85 95.3) (end 138.85 97.95) (width 0.3) (layer F.Cu) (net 5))
 (segment (start 145.5 88.2) (end 145.5 88) (width 0.3) (layer F.Cu) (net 5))
 (segment (start 139.1 95.3) (end 144.4 90) (width 0.3) (layer F.Cu) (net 5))
 (segment (start 144.4 89.3) (end 145.5 88.2) (width 0.3) (layer F.Cu) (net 5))
 (segment (start 144.4 90) (end 144.4 89.3) (width 0.3) (layer F.Cu) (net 5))
 (segment (start 138.85 95.3) (end 139.1 95.3) (width 0.3) (layer F.Cu) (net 5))
 (segment (start 149.58 95) (end 148 95) (width 0.3) (layer F.Cu) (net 7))
 (segment (start 152.5 92.08) (end 149.58 95) (width 0.3) (layer F.Cu) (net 7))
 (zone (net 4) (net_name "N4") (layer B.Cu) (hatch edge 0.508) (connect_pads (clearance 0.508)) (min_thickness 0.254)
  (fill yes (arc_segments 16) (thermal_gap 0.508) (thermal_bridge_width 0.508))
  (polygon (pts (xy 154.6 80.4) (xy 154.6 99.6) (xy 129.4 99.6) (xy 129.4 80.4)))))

